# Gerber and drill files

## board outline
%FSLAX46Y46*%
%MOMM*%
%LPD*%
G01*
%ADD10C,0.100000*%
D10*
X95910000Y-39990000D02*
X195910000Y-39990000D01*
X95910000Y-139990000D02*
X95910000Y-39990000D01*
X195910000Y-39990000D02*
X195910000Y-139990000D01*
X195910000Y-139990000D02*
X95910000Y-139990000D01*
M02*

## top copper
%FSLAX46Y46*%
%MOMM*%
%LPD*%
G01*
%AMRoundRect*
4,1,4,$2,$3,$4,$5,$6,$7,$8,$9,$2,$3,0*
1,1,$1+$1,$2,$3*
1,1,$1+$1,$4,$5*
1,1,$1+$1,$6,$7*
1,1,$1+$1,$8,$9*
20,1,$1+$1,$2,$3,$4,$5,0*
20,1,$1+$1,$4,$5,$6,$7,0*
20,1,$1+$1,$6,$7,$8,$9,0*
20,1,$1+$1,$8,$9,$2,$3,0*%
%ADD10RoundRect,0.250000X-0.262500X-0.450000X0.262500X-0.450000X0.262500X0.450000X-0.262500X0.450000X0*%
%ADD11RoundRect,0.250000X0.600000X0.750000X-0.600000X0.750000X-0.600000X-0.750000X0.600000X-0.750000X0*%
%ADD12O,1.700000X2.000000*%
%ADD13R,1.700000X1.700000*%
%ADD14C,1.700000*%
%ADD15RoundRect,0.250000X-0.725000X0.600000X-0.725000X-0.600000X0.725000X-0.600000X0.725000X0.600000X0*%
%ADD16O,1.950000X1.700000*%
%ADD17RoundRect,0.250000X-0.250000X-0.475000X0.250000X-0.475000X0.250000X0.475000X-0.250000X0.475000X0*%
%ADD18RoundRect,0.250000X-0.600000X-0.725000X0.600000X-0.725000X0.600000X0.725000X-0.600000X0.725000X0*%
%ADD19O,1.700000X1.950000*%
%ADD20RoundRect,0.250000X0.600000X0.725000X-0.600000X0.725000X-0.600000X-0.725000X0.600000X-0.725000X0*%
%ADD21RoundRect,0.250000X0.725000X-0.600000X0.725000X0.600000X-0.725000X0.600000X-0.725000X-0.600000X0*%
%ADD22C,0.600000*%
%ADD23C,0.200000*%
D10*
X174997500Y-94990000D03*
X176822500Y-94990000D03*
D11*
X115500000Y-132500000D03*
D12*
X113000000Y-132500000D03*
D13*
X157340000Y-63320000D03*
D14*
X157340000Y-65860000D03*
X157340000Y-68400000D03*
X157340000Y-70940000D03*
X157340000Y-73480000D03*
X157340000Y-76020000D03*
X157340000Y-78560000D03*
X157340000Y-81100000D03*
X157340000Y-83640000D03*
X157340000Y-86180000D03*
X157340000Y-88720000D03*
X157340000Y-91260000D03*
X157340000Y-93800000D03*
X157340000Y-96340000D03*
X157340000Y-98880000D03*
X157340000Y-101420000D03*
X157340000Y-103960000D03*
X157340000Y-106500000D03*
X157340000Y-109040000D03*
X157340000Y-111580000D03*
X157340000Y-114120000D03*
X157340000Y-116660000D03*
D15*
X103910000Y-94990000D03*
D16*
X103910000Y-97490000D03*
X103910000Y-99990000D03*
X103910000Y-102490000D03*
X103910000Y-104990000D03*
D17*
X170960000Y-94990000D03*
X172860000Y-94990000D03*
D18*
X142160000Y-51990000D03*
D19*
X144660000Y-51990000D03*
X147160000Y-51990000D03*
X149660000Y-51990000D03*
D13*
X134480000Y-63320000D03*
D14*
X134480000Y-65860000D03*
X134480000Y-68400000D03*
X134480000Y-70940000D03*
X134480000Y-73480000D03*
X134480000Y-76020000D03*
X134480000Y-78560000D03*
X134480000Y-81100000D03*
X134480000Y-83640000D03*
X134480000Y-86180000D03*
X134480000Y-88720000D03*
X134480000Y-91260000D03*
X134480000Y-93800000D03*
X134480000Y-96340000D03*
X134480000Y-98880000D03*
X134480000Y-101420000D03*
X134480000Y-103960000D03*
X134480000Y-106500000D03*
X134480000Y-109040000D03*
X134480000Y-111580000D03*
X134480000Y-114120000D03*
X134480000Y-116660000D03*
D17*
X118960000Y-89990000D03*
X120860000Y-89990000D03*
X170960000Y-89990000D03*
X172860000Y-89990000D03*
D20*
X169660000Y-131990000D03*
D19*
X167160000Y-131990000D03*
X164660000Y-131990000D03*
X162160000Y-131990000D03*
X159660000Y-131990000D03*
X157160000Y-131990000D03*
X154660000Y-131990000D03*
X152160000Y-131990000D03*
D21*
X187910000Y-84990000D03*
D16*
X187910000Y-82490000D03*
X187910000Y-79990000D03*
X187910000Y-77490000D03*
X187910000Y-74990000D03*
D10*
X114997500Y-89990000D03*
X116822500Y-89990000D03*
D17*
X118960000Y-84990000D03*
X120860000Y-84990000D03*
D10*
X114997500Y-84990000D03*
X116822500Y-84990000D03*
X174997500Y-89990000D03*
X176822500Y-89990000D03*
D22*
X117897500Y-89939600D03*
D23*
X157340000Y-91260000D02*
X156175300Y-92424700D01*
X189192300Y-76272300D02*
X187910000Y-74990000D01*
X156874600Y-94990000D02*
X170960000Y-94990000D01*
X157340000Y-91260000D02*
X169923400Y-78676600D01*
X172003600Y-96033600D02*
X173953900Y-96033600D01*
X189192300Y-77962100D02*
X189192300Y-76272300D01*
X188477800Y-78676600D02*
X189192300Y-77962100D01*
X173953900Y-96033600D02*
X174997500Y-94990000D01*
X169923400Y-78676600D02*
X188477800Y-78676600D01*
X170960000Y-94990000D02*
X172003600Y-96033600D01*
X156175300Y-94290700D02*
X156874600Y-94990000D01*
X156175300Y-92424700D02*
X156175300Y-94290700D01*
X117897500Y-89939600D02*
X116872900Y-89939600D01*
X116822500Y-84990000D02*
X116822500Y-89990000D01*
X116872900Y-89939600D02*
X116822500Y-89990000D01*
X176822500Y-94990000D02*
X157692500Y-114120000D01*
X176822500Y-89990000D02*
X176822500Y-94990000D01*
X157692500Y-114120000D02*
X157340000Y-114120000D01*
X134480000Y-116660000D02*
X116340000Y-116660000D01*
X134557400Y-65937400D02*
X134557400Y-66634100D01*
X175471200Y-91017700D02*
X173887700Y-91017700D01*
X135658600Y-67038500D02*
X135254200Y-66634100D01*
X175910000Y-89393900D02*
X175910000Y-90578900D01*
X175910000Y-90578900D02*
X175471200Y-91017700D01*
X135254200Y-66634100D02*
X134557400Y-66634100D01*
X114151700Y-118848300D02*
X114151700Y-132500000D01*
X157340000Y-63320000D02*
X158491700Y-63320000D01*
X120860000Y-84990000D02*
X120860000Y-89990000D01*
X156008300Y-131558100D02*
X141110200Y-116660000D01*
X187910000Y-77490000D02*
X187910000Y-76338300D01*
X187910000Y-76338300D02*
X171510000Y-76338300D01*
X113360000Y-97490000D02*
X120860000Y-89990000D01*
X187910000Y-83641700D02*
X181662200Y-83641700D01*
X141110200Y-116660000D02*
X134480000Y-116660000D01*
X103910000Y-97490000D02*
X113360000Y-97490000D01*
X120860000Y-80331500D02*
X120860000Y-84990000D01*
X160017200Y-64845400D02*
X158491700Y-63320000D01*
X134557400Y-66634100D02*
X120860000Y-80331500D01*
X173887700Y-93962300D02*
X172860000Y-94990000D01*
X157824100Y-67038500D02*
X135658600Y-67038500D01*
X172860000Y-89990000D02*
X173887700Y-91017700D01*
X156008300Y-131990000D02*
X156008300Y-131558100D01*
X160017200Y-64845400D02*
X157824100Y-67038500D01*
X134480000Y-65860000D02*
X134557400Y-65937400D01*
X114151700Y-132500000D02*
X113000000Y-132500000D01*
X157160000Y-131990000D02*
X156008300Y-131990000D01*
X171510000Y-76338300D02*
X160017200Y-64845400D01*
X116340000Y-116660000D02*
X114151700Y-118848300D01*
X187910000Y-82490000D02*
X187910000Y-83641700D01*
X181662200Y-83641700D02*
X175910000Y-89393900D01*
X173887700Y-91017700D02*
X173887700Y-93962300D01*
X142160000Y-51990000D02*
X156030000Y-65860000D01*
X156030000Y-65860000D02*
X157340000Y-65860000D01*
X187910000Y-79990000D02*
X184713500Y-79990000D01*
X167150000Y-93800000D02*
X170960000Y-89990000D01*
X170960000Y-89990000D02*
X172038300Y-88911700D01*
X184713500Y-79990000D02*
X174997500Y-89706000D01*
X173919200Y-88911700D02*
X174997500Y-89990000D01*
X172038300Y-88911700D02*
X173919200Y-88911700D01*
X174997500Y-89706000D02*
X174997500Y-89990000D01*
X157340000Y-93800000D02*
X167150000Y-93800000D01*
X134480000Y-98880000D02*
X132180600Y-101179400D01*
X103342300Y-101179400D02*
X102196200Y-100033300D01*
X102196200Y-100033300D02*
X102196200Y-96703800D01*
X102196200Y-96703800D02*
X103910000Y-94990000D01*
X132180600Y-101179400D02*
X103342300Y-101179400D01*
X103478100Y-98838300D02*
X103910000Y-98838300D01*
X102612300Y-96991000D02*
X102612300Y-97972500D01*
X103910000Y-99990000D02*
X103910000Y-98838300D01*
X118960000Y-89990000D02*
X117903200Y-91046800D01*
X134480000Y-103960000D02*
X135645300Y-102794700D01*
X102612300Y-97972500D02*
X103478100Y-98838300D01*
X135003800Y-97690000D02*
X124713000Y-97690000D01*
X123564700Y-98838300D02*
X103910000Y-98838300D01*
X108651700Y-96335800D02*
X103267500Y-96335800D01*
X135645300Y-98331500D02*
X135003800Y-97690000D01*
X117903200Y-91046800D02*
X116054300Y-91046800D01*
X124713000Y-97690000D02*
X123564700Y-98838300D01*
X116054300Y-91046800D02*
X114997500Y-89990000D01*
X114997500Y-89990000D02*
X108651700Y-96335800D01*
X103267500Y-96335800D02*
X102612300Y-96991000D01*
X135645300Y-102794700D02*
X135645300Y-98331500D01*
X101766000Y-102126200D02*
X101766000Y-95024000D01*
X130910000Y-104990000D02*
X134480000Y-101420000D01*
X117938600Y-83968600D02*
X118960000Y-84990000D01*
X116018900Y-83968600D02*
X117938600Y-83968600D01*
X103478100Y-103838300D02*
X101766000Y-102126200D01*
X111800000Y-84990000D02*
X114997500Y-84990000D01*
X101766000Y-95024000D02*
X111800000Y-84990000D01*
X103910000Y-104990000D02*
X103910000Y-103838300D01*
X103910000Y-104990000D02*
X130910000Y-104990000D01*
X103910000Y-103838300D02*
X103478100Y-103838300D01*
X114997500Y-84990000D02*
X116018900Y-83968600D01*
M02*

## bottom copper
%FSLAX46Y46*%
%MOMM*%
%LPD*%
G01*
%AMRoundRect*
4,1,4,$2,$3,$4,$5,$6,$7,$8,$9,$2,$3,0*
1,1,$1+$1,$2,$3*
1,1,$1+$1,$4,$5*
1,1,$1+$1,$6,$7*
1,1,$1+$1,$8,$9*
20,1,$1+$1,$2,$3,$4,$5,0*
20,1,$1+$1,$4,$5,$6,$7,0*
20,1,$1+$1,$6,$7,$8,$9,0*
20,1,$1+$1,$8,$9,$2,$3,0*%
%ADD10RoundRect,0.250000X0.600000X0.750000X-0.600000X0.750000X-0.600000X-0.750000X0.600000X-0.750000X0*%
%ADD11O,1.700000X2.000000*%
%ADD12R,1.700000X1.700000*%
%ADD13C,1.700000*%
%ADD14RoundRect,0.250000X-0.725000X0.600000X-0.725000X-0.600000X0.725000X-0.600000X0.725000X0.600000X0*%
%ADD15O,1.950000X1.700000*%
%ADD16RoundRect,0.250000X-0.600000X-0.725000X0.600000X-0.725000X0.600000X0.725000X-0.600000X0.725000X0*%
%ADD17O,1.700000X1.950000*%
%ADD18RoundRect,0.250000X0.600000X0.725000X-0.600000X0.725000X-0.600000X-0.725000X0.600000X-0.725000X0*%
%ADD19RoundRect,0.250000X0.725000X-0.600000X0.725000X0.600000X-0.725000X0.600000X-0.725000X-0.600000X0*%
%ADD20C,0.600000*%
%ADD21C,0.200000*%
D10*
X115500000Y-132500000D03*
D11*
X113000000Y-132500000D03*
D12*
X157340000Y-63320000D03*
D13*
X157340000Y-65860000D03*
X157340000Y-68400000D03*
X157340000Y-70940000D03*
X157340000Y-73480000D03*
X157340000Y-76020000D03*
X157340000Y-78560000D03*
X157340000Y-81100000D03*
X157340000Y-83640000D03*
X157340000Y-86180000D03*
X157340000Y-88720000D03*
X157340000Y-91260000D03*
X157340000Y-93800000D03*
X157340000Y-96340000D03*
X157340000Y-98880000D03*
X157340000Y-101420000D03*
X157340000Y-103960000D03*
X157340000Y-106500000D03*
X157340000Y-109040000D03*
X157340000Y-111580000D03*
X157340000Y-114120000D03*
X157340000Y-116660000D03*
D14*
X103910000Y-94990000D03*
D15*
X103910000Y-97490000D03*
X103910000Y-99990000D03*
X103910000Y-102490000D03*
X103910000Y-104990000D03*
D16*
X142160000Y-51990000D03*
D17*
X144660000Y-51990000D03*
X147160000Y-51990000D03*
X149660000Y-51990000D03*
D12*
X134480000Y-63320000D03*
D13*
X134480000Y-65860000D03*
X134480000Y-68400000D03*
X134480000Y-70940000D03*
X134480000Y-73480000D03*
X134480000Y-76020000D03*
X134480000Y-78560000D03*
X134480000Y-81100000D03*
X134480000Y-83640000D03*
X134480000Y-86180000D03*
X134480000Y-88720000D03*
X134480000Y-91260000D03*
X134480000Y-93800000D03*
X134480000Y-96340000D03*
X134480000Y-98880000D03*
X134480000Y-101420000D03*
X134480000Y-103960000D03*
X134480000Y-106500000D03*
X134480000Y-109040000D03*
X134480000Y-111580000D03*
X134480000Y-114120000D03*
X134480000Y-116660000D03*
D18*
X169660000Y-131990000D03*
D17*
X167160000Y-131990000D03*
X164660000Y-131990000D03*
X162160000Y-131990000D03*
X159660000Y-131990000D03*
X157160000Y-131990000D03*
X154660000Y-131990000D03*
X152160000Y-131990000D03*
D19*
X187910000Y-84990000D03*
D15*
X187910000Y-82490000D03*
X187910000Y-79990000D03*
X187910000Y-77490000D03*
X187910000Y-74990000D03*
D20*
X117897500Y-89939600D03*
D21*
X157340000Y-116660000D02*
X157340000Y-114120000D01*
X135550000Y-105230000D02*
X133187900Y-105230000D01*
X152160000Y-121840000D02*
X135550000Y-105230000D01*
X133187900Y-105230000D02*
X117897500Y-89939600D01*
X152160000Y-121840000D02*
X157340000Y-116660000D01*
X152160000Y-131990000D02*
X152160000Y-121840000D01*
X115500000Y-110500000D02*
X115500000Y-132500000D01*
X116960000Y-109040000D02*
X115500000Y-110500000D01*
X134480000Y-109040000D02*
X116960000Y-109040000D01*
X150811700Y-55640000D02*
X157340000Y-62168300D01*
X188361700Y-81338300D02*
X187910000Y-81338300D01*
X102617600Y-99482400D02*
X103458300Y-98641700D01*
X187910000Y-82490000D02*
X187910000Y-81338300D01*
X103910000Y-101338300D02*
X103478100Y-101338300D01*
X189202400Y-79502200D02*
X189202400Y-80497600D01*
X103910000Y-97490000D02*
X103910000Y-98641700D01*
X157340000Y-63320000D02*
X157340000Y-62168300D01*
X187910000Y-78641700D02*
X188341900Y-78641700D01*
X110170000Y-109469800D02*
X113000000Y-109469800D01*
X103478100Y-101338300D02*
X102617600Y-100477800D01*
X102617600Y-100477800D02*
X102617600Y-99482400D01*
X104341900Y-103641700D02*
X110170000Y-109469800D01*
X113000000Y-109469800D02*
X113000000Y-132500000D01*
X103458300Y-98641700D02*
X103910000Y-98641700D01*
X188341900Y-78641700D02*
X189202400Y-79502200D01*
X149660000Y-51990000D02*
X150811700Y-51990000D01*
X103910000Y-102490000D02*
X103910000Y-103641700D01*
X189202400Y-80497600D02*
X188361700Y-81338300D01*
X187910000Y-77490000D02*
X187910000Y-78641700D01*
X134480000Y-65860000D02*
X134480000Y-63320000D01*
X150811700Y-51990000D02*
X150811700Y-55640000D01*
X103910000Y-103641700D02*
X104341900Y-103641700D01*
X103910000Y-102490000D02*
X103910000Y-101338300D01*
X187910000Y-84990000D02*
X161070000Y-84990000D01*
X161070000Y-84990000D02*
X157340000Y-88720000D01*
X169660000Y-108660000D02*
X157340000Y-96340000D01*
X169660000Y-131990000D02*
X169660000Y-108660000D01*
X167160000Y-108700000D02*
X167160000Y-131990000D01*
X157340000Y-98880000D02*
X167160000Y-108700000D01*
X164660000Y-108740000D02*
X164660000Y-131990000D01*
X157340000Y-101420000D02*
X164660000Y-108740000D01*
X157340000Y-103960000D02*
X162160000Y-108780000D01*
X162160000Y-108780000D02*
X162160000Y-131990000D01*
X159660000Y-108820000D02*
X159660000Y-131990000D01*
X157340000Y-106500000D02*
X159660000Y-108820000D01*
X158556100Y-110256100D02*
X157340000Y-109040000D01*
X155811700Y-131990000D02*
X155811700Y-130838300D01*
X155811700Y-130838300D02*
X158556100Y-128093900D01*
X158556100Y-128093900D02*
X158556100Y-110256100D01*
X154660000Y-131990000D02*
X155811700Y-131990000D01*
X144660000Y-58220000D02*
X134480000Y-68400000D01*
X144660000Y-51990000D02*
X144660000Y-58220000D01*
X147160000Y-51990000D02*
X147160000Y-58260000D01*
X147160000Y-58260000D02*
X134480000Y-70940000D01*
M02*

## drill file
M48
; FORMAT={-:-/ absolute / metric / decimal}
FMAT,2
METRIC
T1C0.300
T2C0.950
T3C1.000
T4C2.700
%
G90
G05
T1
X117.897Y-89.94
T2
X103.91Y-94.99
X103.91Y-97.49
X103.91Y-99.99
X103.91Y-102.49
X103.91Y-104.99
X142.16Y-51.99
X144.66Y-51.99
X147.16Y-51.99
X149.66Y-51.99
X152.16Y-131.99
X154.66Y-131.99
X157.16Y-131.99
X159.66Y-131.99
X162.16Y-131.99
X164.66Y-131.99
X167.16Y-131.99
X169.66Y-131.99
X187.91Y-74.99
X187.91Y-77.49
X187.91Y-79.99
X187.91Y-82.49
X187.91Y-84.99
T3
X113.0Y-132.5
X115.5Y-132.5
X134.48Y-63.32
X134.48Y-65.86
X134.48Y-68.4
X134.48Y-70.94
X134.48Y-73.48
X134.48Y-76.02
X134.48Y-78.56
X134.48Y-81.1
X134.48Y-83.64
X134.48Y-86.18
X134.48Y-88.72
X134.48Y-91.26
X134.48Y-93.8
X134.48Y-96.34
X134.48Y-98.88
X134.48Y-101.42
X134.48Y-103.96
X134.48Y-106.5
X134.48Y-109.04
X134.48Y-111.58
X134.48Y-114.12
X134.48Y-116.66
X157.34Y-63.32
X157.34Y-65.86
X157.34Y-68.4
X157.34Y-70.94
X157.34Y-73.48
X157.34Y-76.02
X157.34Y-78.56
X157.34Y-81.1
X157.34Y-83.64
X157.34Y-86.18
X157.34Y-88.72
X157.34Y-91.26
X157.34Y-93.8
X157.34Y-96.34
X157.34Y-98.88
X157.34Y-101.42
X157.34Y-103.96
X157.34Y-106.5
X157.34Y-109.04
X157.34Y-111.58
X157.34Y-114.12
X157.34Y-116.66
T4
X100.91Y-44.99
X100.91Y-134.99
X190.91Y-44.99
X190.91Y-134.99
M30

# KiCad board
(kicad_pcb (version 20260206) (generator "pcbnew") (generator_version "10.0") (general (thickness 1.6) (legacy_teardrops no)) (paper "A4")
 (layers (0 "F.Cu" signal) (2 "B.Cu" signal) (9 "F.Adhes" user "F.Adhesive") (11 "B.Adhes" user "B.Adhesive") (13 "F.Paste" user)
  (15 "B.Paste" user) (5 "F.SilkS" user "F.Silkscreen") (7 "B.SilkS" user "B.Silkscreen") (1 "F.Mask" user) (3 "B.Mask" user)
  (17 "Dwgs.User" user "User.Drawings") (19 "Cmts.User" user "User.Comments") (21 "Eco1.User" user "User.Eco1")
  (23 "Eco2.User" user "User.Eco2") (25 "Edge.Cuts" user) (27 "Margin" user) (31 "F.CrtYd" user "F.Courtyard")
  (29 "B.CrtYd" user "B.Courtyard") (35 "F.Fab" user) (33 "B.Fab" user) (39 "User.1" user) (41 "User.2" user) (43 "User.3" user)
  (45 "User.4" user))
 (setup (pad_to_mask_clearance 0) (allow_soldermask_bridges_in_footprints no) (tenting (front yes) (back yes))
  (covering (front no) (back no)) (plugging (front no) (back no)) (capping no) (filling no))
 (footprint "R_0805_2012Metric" (layer "F.Cu") (at 175.91 94.99)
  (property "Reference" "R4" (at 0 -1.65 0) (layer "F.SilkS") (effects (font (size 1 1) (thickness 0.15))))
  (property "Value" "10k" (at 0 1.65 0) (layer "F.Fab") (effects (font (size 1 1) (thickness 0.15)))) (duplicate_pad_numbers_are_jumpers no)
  (pad "1" smd roundrect (at -0.9125 0) (size 1.025 1.4) (layers "F.Cu" "F.Mask" "F.Paste") (roundrect_rratio 0.243902) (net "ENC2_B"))
  (pad "2" smd roundrect (at 0.9125 0) (size 1.025 1.4) (layers "F.Cu" "F.Mask" "F.Paste") (roundrect_rratio 0.243902) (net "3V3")))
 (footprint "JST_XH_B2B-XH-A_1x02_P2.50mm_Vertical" (layer "F.Cu") (at 115.5 132.5 180)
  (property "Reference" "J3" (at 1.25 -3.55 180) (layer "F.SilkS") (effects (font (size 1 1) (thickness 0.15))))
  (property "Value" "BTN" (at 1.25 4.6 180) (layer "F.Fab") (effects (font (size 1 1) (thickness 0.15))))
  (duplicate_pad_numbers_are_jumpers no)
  (pad "1" thru_hole roundrect (at 0 0 180) (size 1.7 2) (drill 1) (layers "*.Cu" "*.Mask") (remove_unused_layers no)
   (roundrect_rratio 0.147059) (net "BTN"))
  (pad "2" thru_hole oval (at 2.5 0 180) (size 1.7 2) (drill 1) (layers "*.Cu" "*.Mask") (remove_unused_layers no) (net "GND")))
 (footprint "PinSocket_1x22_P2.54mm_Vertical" (layer "F.Cu") (at 157.34 63.32)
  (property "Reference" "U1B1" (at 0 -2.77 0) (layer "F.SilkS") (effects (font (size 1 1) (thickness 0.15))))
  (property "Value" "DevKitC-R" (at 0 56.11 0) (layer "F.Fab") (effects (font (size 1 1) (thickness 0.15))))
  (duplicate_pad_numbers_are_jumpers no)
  (pad "1" thru_hole rect (at 0 0) (size 1.7 1.7) (drill 1) (layers "*.Cu" "*.Mask") (remove_unused_layers no) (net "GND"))
  (pad "2" thru_hole circle (at 0 2.54) (size 1.7 1.7) (drill 1) (layers "*.Cu" "*.Mask") (remove_unused_layers no) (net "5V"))
  (pad "3" thru_hole circle (at 0 5.08) (size 1.7 1.7) (drill 1) (layers "*.Cu" "*.Mask") (remove_unused_layers no))
  (pad "4" thru_hole circle (at 0 7.62) (size 1.7 1.7) (drill 1) (layers "*.Cu" "*.Mask") (remove_unused_layers no))
  (pad "5" thru_hole circle (at 0 10.16) (size 1.7 1.7) (drill 1) (layers "*.Cu" "*.Mask") (remove_unused_layers no))
  (pad "6" thru_hole circle (at 0 12.7) (size 1.7 1.7) (drill 1) (layers "*.Cu" "*.Mask") (remove_unused_layers no))
  (pad "7" thru_hole circle (at 0 15.24) (size 1.7 1.7) (drill 1) (layers "*.Cu" "*.Mask") (remove_unused_layers no))
  (pad "8" thru_hole circle (at 0 17.78) (size 1.7 1.7) (drill 1) (layers "*.Cu" "*.Mask") (remove_unused_layers no))
  (pad "9" thru_hole circle (at 0 20.32) (size 1.7 1.7) (drill 1) (layers "*.Cu" "*.Mask") (remove_unused_layers no))
  (pad "10" thru_hole circle (at 0 22.86) (size 1.7 1.7) (drill 1) (layers "*.Cu" "*.Mask") (remove_unused_layers no))
  (pad "11" thru_hole circle (at 0 25.4) (size 1.7 1.7) (drill 1) (layers "*.Cu" "*.Mask") (remove_unused_layers no) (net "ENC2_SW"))
  (pad "12" thru_hole circle (at 0 27.94) (size 1.7 1.7) (drill 1) (layers "*.Cu" "*.Mask") (remove_unused_layers no) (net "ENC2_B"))
  (pad "13" thru_hole circle (at 0 30.48) (size 1.7 1.7) (drill 1) (layers "*.Cu" "*.Mask") (remove_unused_layers no) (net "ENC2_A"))
  (pad "14" thru_hole circle (at 0 33.02) (size 1.7 1.7) (drill 1) (layers "*.Cu" "*.Mask") (remove_unused_layers no) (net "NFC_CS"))
  (pad "15" thru_hole circle (at 0 35.56) (size 1.7 1.7) (drill 1) (layers "*.Cu" "*.Mask") (remove_unused_layers no) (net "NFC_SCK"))
  (pad "16" thru_hole circle (at 0 38.1) (size 1.7 1.7) (drill 1) (layers "*.Cu" "*.Mask") (remove_unused_layers no) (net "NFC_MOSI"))
  (pad "17" thru_hole circle (at 0 40.64) (size 1.7 1.7) (drill 1) (layers "*.Cu" "*.Mask") (remove_unused_layers no) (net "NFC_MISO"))
  (pad "18" thru_hole circle (at 0 43.18) (size 1.7 1.7) (drill 1) (layers "*.Cu" "*.Mask") (remove_unused_layers no) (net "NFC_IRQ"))
  (pad "19" thru_hole circle (at 0 45.72) (size 1.7 1.7) (drill 1) (layers "*.Cu" "*.Mask") (remove_unused_layers no) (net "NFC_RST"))
  (pad "20" thru_hole circle (at 0 48.26) (size 1.7 1.7) (drill 1) (layers "*.Cu" "*.Mask") (remove_unused_layers no))
  (pad "21" thru_hole circle (at 0 50.8) (size 1.7 1.7) (drill 1) (layers "*.Cu" "*.Mask") (remove_unused_layers no) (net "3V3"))
  (pad "22" thru_hole circle (at 0 53.34) (size 1.7 1.7) (drill 1) (layers "*.Cu" "*.Mask") (remove_unused_layers no) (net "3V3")))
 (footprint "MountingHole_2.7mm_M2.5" (layer "F.Cu") (at 190.91 44.99)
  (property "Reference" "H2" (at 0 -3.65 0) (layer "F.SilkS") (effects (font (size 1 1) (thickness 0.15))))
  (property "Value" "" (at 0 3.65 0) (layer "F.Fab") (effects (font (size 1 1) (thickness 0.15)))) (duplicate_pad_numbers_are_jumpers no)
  (pad "" np_thru_hole circle (at 0 0) (size 2.7 2.7) (drill 2.7) (layers "*.Cu" "*.Mask")))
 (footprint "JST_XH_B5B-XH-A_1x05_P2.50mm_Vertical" (layer "F.Cu") (at 103.91 94.99 -90)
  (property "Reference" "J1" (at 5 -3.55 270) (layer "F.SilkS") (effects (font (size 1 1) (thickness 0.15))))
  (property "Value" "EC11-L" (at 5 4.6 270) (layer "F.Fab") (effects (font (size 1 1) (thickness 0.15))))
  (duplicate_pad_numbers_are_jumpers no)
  (pad "1" thru_hole roundrect (at 0 0 270) (size 1.7 1.95) (drill 0.95) (layers "*.Cu" "*.Mask") (remove_unused_layers no)
   (roundrect_rratio 0.147059) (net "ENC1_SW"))
  (pad "2" thru_hole oval (at 2.5 0 270) (size 1.7 1.95) (drill 0.95) (layers "*.Cu" "*.Mask") (remove_unused_layers no) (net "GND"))
  (pad "3" thru_hole oval (at 5 0 270) (size 1.7 1.95) (drill 0.95) (layers "*.Cu" "*.Mask") (remove_unused_layers no) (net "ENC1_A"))
  (pad "4" thru_hole oval (at 7.5 0 270) (size 1.7 1.95) (drill 0.95) (layers "*.Cu" "*.Mask") (remove_unused_layers no) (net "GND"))
  (pad "5" thru_hole oval (at 10 0 270) (size 1.7 1.95) (drill 0.95) (layers "*.Cu" "*.Mask") (remove_unused_layers no) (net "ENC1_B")))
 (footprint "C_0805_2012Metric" (layer "F.Cu") (at 171.91 94.99)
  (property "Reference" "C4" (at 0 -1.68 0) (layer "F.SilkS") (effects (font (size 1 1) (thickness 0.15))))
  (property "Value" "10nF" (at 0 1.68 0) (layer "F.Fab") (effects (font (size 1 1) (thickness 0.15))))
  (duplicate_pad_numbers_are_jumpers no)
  (pad "1" smd roundrect (at -0.95 0) (size 1 1.45) (layers "F.Cu" "F.Mask" "F.Paste") (roundrect_rratio 0.25) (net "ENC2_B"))
  (pad "2" smd roundrect (at 0.95 0) (size 1 1.45) (layers "F.Cu" "F.Mask" "F.Paste") (roundrect_rratio 0.25) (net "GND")))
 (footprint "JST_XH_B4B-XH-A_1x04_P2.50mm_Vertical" (layer "F.Cu") (at 142.16 51.99)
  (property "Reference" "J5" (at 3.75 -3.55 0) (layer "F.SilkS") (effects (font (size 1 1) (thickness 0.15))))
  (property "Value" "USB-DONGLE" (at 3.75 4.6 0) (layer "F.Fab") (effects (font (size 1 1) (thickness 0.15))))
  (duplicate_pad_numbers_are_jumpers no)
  (pad "1" thru_hole roundrect (at 0 0) (size 1.7 1.95) (drill 0.95) (layers "*.Cu" "*.Mask") (remove_unused_layers no)
   (roundrect_rratio 0.147059) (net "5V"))
  (pad "2" thru_hole oval (at 2.5 0) (size 1.7 1.95) (drill 0.95) (layers "*.Cu" "*.Mask") (remove_unused_layers no) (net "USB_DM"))
  (pad "3" thru_hole oval (at 5 0) (size 1.7 1.95) (drill 0.95) (layers "*.Cu" "*.Mask") (remove_unused_layers no) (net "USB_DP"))
  (pad "4" thru_hole oval (at 7.5 0) (size 1.7 1.95) (drill 0.95) (layers "*.Cu" "*.Mask") (remove_unused_layers no) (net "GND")))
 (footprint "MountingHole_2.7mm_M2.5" (layer "F.Cu") (at 100.91 134.99)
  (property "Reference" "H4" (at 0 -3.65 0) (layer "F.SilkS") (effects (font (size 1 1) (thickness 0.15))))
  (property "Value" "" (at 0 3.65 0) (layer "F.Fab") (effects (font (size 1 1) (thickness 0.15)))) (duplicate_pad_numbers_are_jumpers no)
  (pad "" np_thru_hole circle (at 0 0) (size 2.7 2.7) (drill 2.7) (layers "*.Cu" "*.Mask")))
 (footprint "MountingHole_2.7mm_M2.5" (layer "F.Cu") (at 100.91 44.99)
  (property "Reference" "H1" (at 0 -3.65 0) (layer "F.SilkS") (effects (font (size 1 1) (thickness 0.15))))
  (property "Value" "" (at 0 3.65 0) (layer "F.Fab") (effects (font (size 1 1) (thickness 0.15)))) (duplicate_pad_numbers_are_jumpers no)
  (pad "" np_thru_hole circle (at 0 0) (size 2.7 2.7) (drill 2.7) (layers "*.Cu" "*.Mask")))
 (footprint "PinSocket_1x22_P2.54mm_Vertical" (layer "F.Cu") (at 134.48 63.32)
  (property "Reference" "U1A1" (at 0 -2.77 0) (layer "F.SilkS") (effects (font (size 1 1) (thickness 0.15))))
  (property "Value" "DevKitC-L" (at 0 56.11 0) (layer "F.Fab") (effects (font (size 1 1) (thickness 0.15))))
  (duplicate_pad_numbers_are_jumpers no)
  (pad "1" thru_hole rect (at 0 0) (size 1.7 1.7) (drill 1) (layers "*.Cu" "*.Mask") (remove_unused_layers no) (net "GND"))
  (pad "2" thru_hole circle (at 0 2.54) (size 1.7 1.7) (drill 1) (layers "*.Cu" "*.Mask") (remove_unused_layers no) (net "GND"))
  (pad "3" thru_hole circle (at 0 5.08) (size 1.7 1.7) (drill 1) (layers "*.Cu" "*.Mask") (remove_unused_layers no) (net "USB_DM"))
  (pad "4" thru_hole circle (at 0 7.62) (size 1.7 1.7) (drill 1) (layers "*.Cu" "*.Mask") (remove_unused_layers no) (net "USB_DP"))
  (pad "5" thru_hole circle (at 0 10.16) (size 1.7 1.7) (drill 1) (layers "*.Cu" "*.Mask") (remove_unused_layers no))
  (pad "6" thru_hole circle (at 0 12.7) (size 1.7 1.7) (drill 1) (layers "*.Cu" "*.Mask") (remove_unused_layers no))
  (pad "7" thru_hole circle (at 0 15.24) (size 1.7 1.7) (drill 1) (layers "*.Cu" "*.Mask") (remove_unused_layers no))
  (pad "8" thru_hole circle (at 0 17.78) (size 1.7 1.7) (drill 1) (layers "*.Cu" "*.Mask") (remove_unused_layers no))
  (pad "9" thru_hole circle (at 0 20.32) (size 1.7 1.7) (drill 1) (layers "*.Cu" "*.Mask") (remove_unused_layers no))
  (pad "10" thru_hole circle (at 0 22.86) (size 1.7 1.7) (drill 1) (layers "*.Cu" "*.Mask") (remove_unused_layers no))
  (pad "11" thru_hole circle (at 0 25.4) (size 1.7 1.7) (drill 1) (layers "*.Cu" "*.Mask") (remove_unused_layers no))
  (pad "12" thru_hole circle (at 0 27.94) (size 1.7 1.7) (drill 1) (layers "*.Cu" "*.Mask") (remove_unused_layers no))
  (pad "13" thru_hole circle (at 0 30.48) (size 1.7 1.7) (drill 1) (layers "*.Cu" "*.Mask") (remove_unused_layers no))
  (pad "14" thru_hole circle (at 0 33.02) (size 1.7 1.7) (drill 1) (layers "*.Cu" "*.Mask") (remove_unused_layers no))
  (pad "15" thru_hole circle (at 0 35.56) (size 1.7 1.7) (drill 1) (layers "*.Cu" "*.Mask") (remove_unused_layers no) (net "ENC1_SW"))
  (pad "16" thru_hole circle (at 0 38.1) (size 1.7 1.7) (drill 1) (layers "*.Cu" "*.Mask") (remove_unused_layers no) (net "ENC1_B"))
  (pad "17" thru_hole circle (at 0 40.64) (size 1.7 1.7) (drill 1) (layers "*.Cu" "*.Mask") (remove_unused_layers no) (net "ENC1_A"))
  (pad "18" thru_hole circle (at 0 43.18) (size 1.7 1.7) (drill 1) (layers "*.Cu" "*.Mask") (remove_unused_layers no))
  (pad "19" thru_hole circle (at 0 45.72) (size 1.7 1.7) (drill 1) (layers "*.Cu" "*.Mask") (remove_unused_layers no) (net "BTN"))
  (pad "20" thru_hole circle (at 0 48.26) (size 1.7 1.7) (drill 1) (layers "*.Cu" "*.Mask") (remove_unused_layers no))
  (pad "21" thru_hole circle (at 0 50.8) (size 1.7 1.7) (drill 1) (layers "*.Cu" "*.Mask") (remove_unused_layers no))
  (pad "22" thru_hole circle (at 0 53.34) (size 1.7 1.7) (drill 1) (layers "*.Cu" "*.Mask") (remove_unused_layers no) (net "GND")))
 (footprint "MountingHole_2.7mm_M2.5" (layer "F.Cu") (at 190.91 134.99)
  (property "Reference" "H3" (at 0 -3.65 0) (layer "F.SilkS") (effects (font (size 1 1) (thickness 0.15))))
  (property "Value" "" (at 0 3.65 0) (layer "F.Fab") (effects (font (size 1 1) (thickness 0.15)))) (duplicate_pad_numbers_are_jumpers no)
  (pad "" np_thru_hole circle (at 0 0) (size 2.7 2.7) (drill 2.7) (layers "*.Cu" "*.Mask")))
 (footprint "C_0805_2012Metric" (layer "F.Cu") (at 119.91 89.99)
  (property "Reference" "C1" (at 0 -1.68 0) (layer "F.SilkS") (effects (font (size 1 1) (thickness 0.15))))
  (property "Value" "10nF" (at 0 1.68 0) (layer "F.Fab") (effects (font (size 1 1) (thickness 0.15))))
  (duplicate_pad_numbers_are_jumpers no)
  (pad "1" smd roundrect (at -0.95 0) (size 1 1.45) (layers "F.Cu" "F.Mask" "F.Paste") (roundrect_rratio 0.25) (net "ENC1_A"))
  (pad "2" smd roundrect (at 0.95 0) (size 1 1.45) (layers "F.Cu" "F.Mask" "F.Paste") (roundrect_rratio 0.25) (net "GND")))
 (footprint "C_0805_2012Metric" (layer "F.Cu") (at 171.91 89.99)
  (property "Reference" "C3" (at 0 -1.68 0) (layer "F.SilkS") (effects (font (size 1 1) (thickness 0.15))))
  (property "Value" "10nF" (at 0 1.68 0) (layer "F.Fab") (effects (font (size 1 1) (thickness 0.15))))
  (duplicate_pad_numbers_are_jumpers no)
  (pad "1" smd roundrect (at -0.95 0) (size 1 1.45) (layers "F.Cu" "F.Mask" "F.Paste") (roundrect_rratio 0.25) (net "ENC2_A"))
  (pad "2" smd roundrect (at 0.95 0) (size 1 1.45) (layers "F.Cu" "F.Mask" "F.Paste") (roundrect_rratio 0.25) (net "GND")))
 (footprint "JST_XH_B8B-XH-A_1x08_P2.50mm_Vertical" (layer "F.Cu") (at 169.66 131.99 180)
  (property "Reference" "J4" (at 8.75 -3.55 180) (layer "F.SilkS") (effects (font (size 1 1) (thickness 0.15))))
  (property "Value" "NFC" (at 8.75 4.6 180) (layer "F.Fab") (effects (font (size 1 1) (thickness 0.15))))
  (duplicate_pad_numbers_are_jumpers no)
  (pad "1" thru_hole roundrect (at 0 0 180) (size 1.7 1.95) (drill 0.95) (layers "*.Cu" "*.Mask") (remove_unused_layers no)
   (roundrect_rratio 0.147059) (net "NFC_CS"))
  (pad "2" thru_hole oval (at 2.5 0 180) (size 1.7 1.95) (drill 0.95) (layers "*.Cu" "*.Mask") (remove_unused_layers no) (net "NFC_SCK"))
  (pad "3" thru_hole oval (at 5 0 180) (size 1.7 1.95) (drill 0.95) (layers "*.Cu" "*.Mask") (remove_unused_layers no) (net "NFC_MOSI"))
  (pad "4" thru_hole oval (at 7.5 0 180) (size 1.7 1.95) (drill 0.95) (layers "*.Cu" "*.Mask") (remove_unused_layers no) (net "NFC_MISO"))
  (pad "5" thru_hole oval (at 10 0 180) (size 1.7 1.95) (drill 0.95) (layers "*.Cu" "*.Mask") (remove_unused_layers no) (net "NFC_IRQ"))
  (pad "6" thru_hole oval (at 12.5 0 180) (size 1.7 1.95) (drill 0.95) (layers "*.Cu" "*.Mask") (remove_unused_layers no) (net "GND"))
  (pad "7" thru_hole oval (at 15 0 180) (size 1.7 1.95) (drill 0.95) (layers "*.Cu" "*.Mask") (remove_unused_layers no) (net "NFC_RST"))
  (pad "8" thru_hole oval (at 17.5 0 180) (size 1.7 1.95) (drill 0.95) (layers "*.Cu" "*.Mask") (remove_unused_layers no) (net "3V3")))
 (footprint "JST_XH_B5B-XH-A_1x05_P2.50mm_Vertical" (layer "F.Cu") (at 187.91 84.99 90)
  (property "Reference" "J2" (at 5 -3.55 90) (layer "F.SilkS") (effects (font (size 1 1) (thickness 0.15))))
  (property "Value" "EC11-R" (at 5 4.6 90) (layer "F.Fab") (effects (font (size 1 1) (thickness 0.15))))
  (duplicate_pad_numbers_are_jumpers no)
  (pad "1" thru_hole roundrect (at 0 0 90) (size 1.7 1.95) (drill 0.95) (layers "*.Cu" "*.Mask") (remove_unused_layers no)
   (roundrect_rratio 0.147059) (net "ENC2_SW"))
  (pad "2" thru_hole oval (at 2.5 0 90) (size 1.7 1.95) (drill 0.95) (layers "*.Cu" "*.Mask") (remove_unused_layers no) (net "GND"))
  (pad "3" thru_hole oval (at 5 0 90) (size 1.7 1.95) (drill 0.95) (layers "*.Cu" "*.Mask") (remove_unused_layers no) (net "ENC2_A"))
  (pad "4" thru_hole oval (at 7.5 0 90) (size 1.7 1.95) (drill 0.95) (layers "*.Cu" "*.Mask") (remove_unused_layers no) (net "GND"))
  (pad "5" thru_hole oval (at 10 0 90) (size 1.7 1.95) (drill 0.95) (layers "*.Cu" "*.Mask") (remove_unused_layers no) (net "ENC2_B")))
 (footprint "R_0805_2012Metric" (layer "F.Cu") (at 115.91 89.99)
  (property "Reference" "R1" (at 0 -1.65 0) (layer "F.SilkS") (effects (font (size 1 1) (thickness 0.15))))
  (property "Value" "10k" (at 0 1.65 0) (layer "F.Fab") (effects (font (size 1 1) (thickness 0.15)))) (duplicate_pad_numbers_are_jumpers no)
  (pad "1" smd roundrect (at -0.9125 0) (size 1.025 1.4) (layers "F.Cu" "F.Mask" "F.Paste") (roundrect_rratio 0.243902) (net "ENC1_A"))
  (pad "2" smd roundrect (at 0.9125 0) (size 1.025 1.4) (layers "F.Cu" "F.Mask" "F.Paste") (roundrect_rratio 0.243902) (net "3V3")))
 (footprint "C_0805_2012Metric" (layer "F.Cu") (at 119.91 84.99)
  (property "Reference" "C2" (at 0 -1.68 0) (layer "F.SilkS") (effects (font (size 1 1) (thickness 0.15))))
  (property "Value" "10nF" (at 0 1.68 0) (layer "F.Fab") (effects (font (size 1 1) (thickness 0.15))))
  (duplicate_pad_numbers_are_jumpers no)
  (pad "1" smd roundrect (at -0.95 0) (size 1 1.45) (layers "F.Cu" "F.Mask" "F.Paste") (roundrect_rratio 0.25) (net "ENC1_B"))
  (pad "2" smd roundrect (at 0.95 0) (size 1 1.45) (layers "F.Cu" "F.Mask" "F.Paste") (roundrect_rratio 0.25) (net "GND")))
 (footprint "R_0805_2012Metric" (layer "F.Cu") (at 115.91 84.99)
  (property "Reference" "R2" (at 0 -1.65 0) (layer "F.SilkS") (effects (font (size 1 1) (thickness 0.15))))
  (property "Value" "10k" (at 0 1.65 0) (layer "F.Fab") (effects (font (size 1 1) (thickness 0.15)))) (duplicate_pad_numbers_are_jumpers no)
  (pad "1" smd roundrect (at -0.9125 0) (size 1.025 1.4) (layers "F.Cu" "F.Mask" "F.Paste") (roundrect_rratio 0.243902) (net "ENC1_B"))
  (pad "2" smd roundrect (at 0.9125 0) (size 1.025 1.4) (layers "F.Cu" "F.Mask" "F.Paste") (roundrect_rratio 0.243902) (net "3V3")))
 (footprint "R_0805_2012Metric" (layer "F.Cu") (at 175.91 89.99)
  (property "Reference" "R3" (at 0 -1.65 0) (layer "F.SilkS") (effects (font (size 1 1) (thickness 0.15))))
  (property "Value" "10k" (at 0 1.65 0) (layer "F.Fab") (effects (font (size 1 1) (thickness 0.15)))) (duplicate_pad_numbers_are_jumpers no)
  (pad "1" smd roundrect (at -0.9125 0) (size 1.025 1.4) (layers "F.Cu" "F.Mask" "F.Paste") (roundrect_rratio 0.243902) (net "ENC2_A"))
  (pad "2" smd roundrect (at 0.9125 0) (size 1.025 1.4) (layers "F.Cu" "F.Mask" "F.Paste") (roundrect_rratio 0.243902) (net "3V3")))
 (gr_line (start 95.91 39.99) (end 195.91 39.99) (stroke (width 0.1) (type default)) (layer "Edge.Cuts"))
 (gr_line (start 95.91 139.99) (end 95.91 39.99) (stroke (width 0.1) (type default)) (layer "Edge.Cuts"))
 (gr_line (start 195.91 39.99) (end 195.91 139.99) (stroke (width 0.1) (type default)) (layer "Edge.Cuts"))
 (gr_line (start 195.91 139.99) (end 95.91 139.99) (stroke (width 0.1) (type default)) (layer "Edge.Cuts"))
 (segment (start 157.34 91.26) (end 156.1753 92.4247) (width 0.2) (layer "F.Cu") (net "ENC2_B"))
 (segment (start 189.1923 76.2723) (end 187.91 74.99) (width 0.2) (layer "F.Cu") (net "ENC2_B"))
 (segment (start 156.8746 94.99) (end 170.96 94.99) (width 0.2) (layer "F.Cu") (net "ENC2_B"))
 (segment (start 157.34 91.26) (end 169.9234 78.6766) (width 0.2) (layer "F.Cu") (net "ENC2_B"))
 (segment (start 172.0036 96.0336) (end 173.9539 96.0336) (width 0.2) (layer "F.Cu") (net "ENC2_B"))
 (segment (start 189.1923 77.9621) (end 189.1923 76.2723) (width 0.2) (layer "F.Cu") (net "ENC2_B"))
 (segment (start 188.4778 78.6766) (end 189.1923 77.9621) (width 0.2) (layer "F.Cu") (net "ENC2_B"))
 (segment (start 173.9539 96.0336) (end 174.9975 94.99) (width 0.2) (layer "F.Cu") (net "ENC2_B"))
 (segment (start 169.9234 78.6766) (end 188.4778 78.6766) (width 0.2) (layer "F.Cu") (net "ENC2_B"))
 (segment (start 170.96 94.99) (end 172.0036 96.0336) (width 0.2) (layer "F.Cu") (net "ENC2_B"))
 (segment (start 156.1753 94.2907) (end 156.8746 94.99) (width 0.2) (layer "F.Cu") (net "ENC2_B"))
 (segment (start 156.1753 92.4247) (end 156.1753 94.2907) (width 0.2) (layer "F.Cu") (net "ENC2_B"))
 (segment (start 117.8975 89.9396) (end 116.8729 89.9396) (width 0.2) (layer "F.Cu") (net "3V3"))
 (segment (start 116.8225 84.99) (end 116.8225 89.99) (width 0.2) (layer "F.Cu") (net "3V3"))
 (segment (start 116.8729 89.9396) (end 116.8225 89.99) (width 0.2) (layer "F.Cu") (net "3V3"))
 (segment (start 176.8225 94.99) (end 157.6925 114.12) (width 0.2) (layer "F.Cu") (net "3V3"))
 (segment (start 176.8225 89.99) (end 176.8225 94.99) (width 0.2) (layer "F.Cu") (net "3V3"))
 (segment (start 157.6925 114.12) (end 157.34 114.12) (width 0.2) (layer "F.Cu") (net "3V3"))
 (via (at 117.8975 89.9396) (size 0.6) (drill 0.3) (layers "F.Cu" "B.Cu") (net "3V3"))
 (segment (start 157.34 116.66) (end 157.34 114.12) (width 0.2) (layer "B.Cu") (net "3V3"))
 (segment (start 135.55 105.23) (end 133.1879 105.23) (width 0.2) (layer "B.Cu") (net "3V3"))
 (segment (start 152.16 121.84) (end 135.55 105.23) (width 0.2) (layer "B.Cu") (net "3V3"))
 (segment (start 133.1879 105.23) (end 117.8975 89.9396) (width 0.2) (layer "B.Cu") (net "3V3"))
 (segment (start 152.16 121.84) (end 157.34 116.66) (width 0.2) (layer "B.Cu") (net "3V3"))
 (segment (start 152.16 131.99) (end 152.16 121.84) (width 0.2) (layer "B.Cu") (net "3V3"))
 (segment (start 115.5 110.5) (end 115.5 132.5) (width 0.2) (layer "B.Cu") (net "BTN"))
 (segment (start 116.96 109.04) (end 115.5 110.5) (width 0.2) (layer "B.Cu") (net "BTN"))
 (segment (start 134.48 109.04) (end 116.96 109.04) (width 0.2) (layer "B.Cu") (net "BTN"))
 (segment (start 134.48 116.66) (end 116.34 116.66) (width 0.2) (layer "F.Cu") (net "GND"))
 (segment (start 134.5574 65.9374) (end 134.5574 66.6341) (width 0.2) (layer "F.Cu") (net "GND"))
 (segment (start 175.4712 91.0177) (end 173.8877 91.0177) (width 0.2) (layer "F.Cu") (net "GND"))
 (segment (start 135.6586 67.0385) (end 135.2542 66.6341) (width 0.2) (layer "F.Cu") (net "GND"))
 (segment (start 175.91 89.3939) (end 175.91 90.5789) (width 0.2) (layer "F.Cu") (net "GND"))
 (segment (start 175.91 90.5789) (end 175.4712 91.0177) (width 0.2) (layer "F.Cu") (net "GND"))
 (segment (start 135.2542 66.6341) (end 134.5574 66.6341) (width 0.2) (layer "F.Cu") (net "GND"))
 (segment (start 114.1517 118.8483) (end 114.1517 132.5) (width 0.2) (layer "F.Cu") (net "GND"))
 (segment (start 157.34 63.32) (end 158.4917 63.32) (width 0.2) (layer "F.Cu") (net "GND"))
 (segment (start 120.86 84.99) (end 120.86 89.99) (width 0.2) (layer "F.Cu") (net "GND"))
 (segment (start 156.0083 131.5581) (end 141.1102 116.66) (width 0.2) (layer "F.Cu") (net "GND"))
 (segment (start 187.91 77.49) (end 187.91 76.3383) (width 0.2) (layer "F.Cu") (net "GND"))
 (segment (start 187.91 76.3383) (end 171.51 76.3383) (width 0.2) (layer "F.Cu") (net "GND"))
 (segment (start 113.36 97.49) (end 120.86 89.99) (width 0.2) (layer "F.Cu") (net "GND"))
 (segment (start 187.91 83.6417) (end 181.6622 83.6417) (width 0.2) (layer "F.Cu") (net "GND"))
 (segment (start 141.1102 116.66) (end 134.48 116.66) (width 0.2) (layer "F.Cu") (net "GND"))
 (segment (start 103.91 97.49) (end 113.36 97.49) (width 0.2) (layer "F.Cu") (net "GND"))
 (segment (start 120.86 80.3315) (end 120.86 84.99) (width 0.2) (layer "F.Cu") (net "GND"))
 (segment (start 160.0172 64.8454) (end 158.4917 63.32) (width 0.2) (layer "F.Cu") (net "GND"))
 (segment (start 134.5574 66.6341) (end 120.86 80.3315) (width 0.2) (layer "F.Cu") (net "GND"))
 (segment (start 173.8877 93.9623) (end 172.86 94.99) (width 0.2) (layer "F.Cu") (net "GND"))
 (segment (start 157.8241 67.0385) (end 135.6586 67.0385) (width 0.2) (layer "F.Cu") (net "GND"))
 (segment (start 172.86 89.99) (end 173.8877 91.0177) (width 0.2) (layer "F.Cu") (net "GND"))
 (segment (start 156.0083 131.99) (end 156.0083 131.5581) (width 0.2) (layer "F.Cu") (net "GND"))
 (segment (start 160.0172 64.8454) (end 157.8241 67.0385) (width 0.2) (layer "F.Cu") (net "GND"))
 (segment (start 134.48 65.86) (end 134.5574 65.9374) (width 0.2) (layer "F.Cu") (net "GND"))
 (segment (start 114.1517 132.5) (end 113 132.5) (width 0.2) (layer "F.Cu") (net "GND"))
 (segment (start 157.16 131.99) (end 156.0083 131.99) (width 0.2) (layer "F.Cu") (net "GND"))
 (segment (start 171.51 76.3383) (end 160.0172 64.8454) (width 0.2) (layer "F.Cu") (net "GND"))
 (segment (start 116.34 116.66) (end 114.1517 118.8483) (width 0.2) (layer "F.Cu") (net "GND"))
 (segment (start 187.91 82.49) (end 187.91 83.6417) (width 0.2) (layer "F.Cu") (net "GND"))
 (segment (start 181.6622 83.6417) (end 175.91 89.3939) (width 0.2) (layer "F.Cu") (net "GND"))
 (segment (start 173.8877 91.0177) (end 173.8877 93.9623) (width 0.2) (layer "F.Cu") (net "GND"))
 (segment (start 150.8117 55.64) (end 157.34 62.1683) (width 0.2) (layer "B.Cu") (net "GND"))
 (segment (start 188.3617 81.3383) (end 187.91 81.3383) (width 0.2) (layer "B.Cu") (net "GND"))
 (segment (start 102.6176 99.4824) (end 103.4583 98.6417) (width 0.2) (layer "B.Cu") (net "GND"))
 (segment (start 187.91 82.49) (end 187.91 81.3383) (width 0.2) (layer "B.Cu") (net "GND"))
 (segment (start 103.91 101.3383) (end 103.4781 101.3383) (width 0.2) (layer "B.Cu") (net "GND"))
 (segment (start 189.2024 79.5022) (end 189.2024 80.4976) (width 0.2) (layer "B.Cu") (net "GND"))
 (segment (start 103.91 97.49) (end 103.91 98.6417) (width 0.2) (layer "B.Cu") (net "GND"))
 (segment (start 157.34 63.32) (end 157.34 62.1683) (width 0.2) (layer "B.Cu") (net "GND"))
 (segment (start 187.91 78.6417) (end 188.3419 78.6417) (width 0.2) (layer "B.Cu") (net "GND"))
 (segment (start 110.17 109.4698) (end 113 109.4698) (width 0.2) (layer "B.Cu") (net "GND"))
 (segment (start 103.4781 101.3383) (end 102.6176 100.4778) (width 0.2) (layer "B.Cu") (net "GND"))
 (segment (start 102.6176 100.4778) (end 102.6176 99.4824) (width 0.2) (layer "B.Cu") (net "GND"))
 (segment (start 104.3419 103.6417) (end 110.17 109.4698) (width 0.2) (layer "B.Cu") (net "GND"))
 (segment (start 113 109.4698) (end 113 132.5) (width 0.2) (layer "B.Cu") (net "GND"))
 (segment (start 103.4583 98.6417) (end 103.91 98.6417) (width 0.2) (layer "B.Cu") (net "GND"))
 (segment (start 188.3419 78.6417) (end 189.2024 79.5022) (width 0.2) (layer "B.Cu") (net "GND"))
 (segment (start 149.66 51.99) (end 150.8117 51.99) (width 0.2) (layer "B.Cu") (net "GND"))
 (segment (start 103.91 102.49) (end 103.91 103.6417) (width 0.2) (layer "B.Cu") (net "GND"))
 (segment (start 189.2024 80.4976) (end 188.3617 81.3383) (width 0.2) (layer "B.Cu") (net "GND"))
 (segment (start 187.91 77.49) (end 187.91 78.6417) (width 0.2) (layer "B.Cu") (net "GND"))
 (segment (start 134.48 65.86) (end 134.48 63.32) (width 0.2) (layer "B.Cu") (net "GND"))
 (segment (start 150.8117 51.99) (end 150.8117 55.64) (width 0.2) (layer "B.Cu") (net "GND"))
 (segment (start 103.91 103.6417) (end 104.3419 103.6417) (width 0.2) (layer "B.Cu") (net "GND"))
 (segment (start 103.91 102.49) (end 103.91 101.3383) (width 0.2) (layer "B.Cu") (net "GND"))
 (segment (start 142.16 51.99) (end 156.03 65.86) (width 0.2) (layer "F.Cu") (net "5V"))
 (segment (start 156.03 65.86) (end 157.34 65.86) (width 0.2) (layer "F.Cu") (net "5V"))
 (segment (start 187.91 84.99) (end 161.07 84.99) (width 0.2) (layer "B.Cu") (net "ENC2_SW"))
 (segment (start 161.07 84.99) (end 157.34 88.72) (width 0.2) (layer "B.Cu") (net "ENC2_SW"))
 (segment (start 187.91 79.99) (end 184.7135 79.99) (width 0.2) (layer "F.Cu") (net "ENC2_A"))
 (segment (start 167.15 93.8) (end 170.96 89.99) (width 0.2) (layer "F.Cu") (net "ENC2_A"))
 (segment (start 170.96 89.99) (end 172.0383 88.9117) (width 0.2) (layer "F.Cu") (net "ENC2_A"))
 (segment (start 184.7135 79.99) (end 174.9975 89.706) (width 0.2) (layer "F.Cu") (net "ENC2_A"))
 (segment (start 173.9192 88.9117) (end 174.9975 89.99) (width 0.2) (layer "F.Cu") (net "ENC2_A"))
 (segment (start 172.0383 88.9117) (end 173.9192 88.9117) (width 0.2) (layer "F.Cu") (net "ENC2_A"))
 (segment (start 174.9975 89.706) (end 174.9975 89.99) (width 0.2) (layer "F.Cu") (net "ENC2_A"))
 (segment (start 157.34 93.8) (end 167.15 93.8) (width 0.2) (layer "F.Cu") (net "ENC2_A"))
 (segment (start 169.66 108.66) (end 157.34 96.34) (width 0.2) (layer "B.Cu") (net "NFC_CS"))
 (segment (start 169.66 131.99) (end 169.66 108.66) (width 0.2) (layer "B.Cu") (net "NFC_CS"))
 (segment (start 167.16 108.7) (end 167.16 131.99) (width 0.2) (layer "B.Cu") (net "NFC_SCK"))
 (segment (start 157.34 98.88) (end 167.16 108.7) (width 0.2) (layer "B.Cu") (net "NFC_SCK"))
 (segment (start 164.66 108.74) (end 164.66 131.99) (width 0.2) (layer "B.Cu") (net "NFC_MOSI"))
 (segment (start 157.34 101.42) (end 164.66 108.74) (width 0.2) (layer "B.Cu") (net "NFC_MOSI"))
 (segment (start 157.34 103.96) (end 162.16 108.78) (width 0.2) (layer "B.Cu") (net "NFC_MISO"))
 (segment (start 162.16 108.78) (end 162.16 131.99) (width 0.2) (layer "B.Cu") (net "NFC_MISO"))
 (segment (start 159.66 108.82) (end 159.66 131.99) (width 0.2) (layer "B.Cu") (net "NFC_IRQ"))
 (segment (start 157.34 106.5) (end 159.66 108.82) (width 0.2) (layer "B.Cu") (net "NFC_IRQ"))
 (segment (start 158.5561 110.2561) (end 157.34 109.04) (width 0.2) (layer "B.Cu") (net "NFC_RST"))
 (segment (start 155.8117 131.99) (end 155.8117 130.8383) (width 0.2) (layer "B.Cu") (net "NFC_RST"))
 (segment (start 155.8117 130.8383) (end 158.5561 128.0939) (width 0.2) (layer "B.Cu") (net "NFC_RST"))
 (segment (start 158.5561 128.0939) (end 158.5561 110.2561) (width 0.2) (layer "B.Cu") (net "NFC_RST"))
 (segment (start 154.66 131.99) (end 155.8117 131.99) (width 0.2) (layer "B.Cu") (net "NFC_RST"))
 (segment (start 134.48 98.88) (end 132.1806 101.1794) (width 0.2) (layer "F.Cu") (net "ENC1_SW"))
 (segment (start 103.3423 101.1794) (end 102.1962 100.0333) (width 0.2) (layer "F.Cu") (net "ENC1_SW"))
 (segment (start 102.1962 100.0333) (end 102.1962 96.7038) (width 0.2) (layer "F.Cu") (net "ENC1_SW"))
 (segment (start 102.1962 96.7038) (end 103.91 94.99) (width 0.2) (layer "F.Cu") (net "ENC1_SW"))
 (segment (start 132.1806 101.1794) (end 103.3423 101.1794) (width 0.2) (layer "F.Cu") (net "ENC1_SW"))
 (segment (start 103.4781 98.8383) (end 103.91 98.8383) (width 0.2) (layer "F.Cu") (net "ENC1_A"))
 (segment (start 102.6123 96.991) (end 102.6123 97.9725) (width 0.2) (layer "F.Cu") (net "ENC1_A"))
 (segment (start 103.91 99.99) (end 103.91 98.8383) (width 0.2) (layer "F.Cu") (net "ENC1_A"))
 (segment (start 118.96 89.99) (end 117.9032 91.0468) (width 0.2) (layer "F.Cu") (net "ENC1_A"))
 (segment (start 134.48 103.96) (end 135.6453 102.7947) (width 0.2) (layer "F.Cu") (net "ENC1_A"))
 (segment (start 102.6123 97.9725) (end 103.4781 98.8383) (width 0.2) (layer "F.Cu") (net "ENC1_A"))
 (segment (start 135.0038 97.69) (end 124.713 97.69) (width 0.2) (layer "F.Cu") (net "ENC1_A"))
 (segment (start 123.5647 98.8383) (end 103.91 98.8383) (width 0.2) (layer "F.Cu") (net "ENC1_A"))
 (segment (start 108.6517 96.3358) (end 103.2675 96.3358) (width 0.2) (layer "F.Cu") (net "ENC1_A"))
 (segment (start 135.6453 98.3315) (end 135.0038 97.69) (width 0.2) (layer "F.Cu") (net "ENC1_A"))
 (segment (start 117.9032 91.0468) (end 116.0543 91.0468) (width 0.2) (layer "F.Cu") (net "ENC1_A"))
 (segment (start 124.713 97.69) (end 123.5647 98.8383) (width 0.2) (layer "F.Cu") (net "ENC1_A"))
 (segment (start 116.0543 91.0468) (end 114.9975 89.99) (width 0.2) (layer "F.Cu") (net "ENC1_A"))
 (segment (start 114.9975 89.99) (end 108.6517 96.3358) (width 0.2) (layer "F.Cu") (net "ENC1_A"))
 (segment (start 103.2675 96.3358) (end 102.6123 96.991) (width 0.2) (layer "F.Cu") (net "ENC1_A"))
 (segment (start 135.6453 102.7947) (end 135.6453 98.3315) (width 0.2) (layer "F.Cu") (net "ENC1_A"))
 (segment (start 101.766 102.1262) (end 101.766 95.024) (width 0.2) (layer "F.Cu") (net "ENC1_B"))
 (segment (start 130.91 104.99) (end 134.48 101.42) (width 0.2) (layer "F.Cu") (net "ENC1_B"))
 (segment (start 117.9386 83.9686) (end 118.96 84.99) (width 0.2) (layer "F.Cu") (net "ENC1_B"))
 (segment (start 116.0189 83.9686) (end 117.9386 83.9686) (width 0.2) (layer "F.Cu") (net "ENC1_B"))
 (segment (start 103.4781 103.8383) (end 101.766 102.1262) (width 0.2) (layer "F.Cu") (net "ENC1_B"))
 (segment (start 111.8 84.99) (end 114.9975 84.99) (width 0.2) (layer "F.Cu") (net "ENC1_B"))
 (segment (start 101.766 95.024) (end 111.8 84.99) (width 0.2) (layer "F.Cu") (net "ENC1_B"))
 (segment (start 103.91 104.99) (end 103.91 103.8383) (width 0.2) (layer "F.Cu") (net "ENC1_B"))
 (segment (start 103.91 104.99) (end 130.91 104.99) (width 0.2) (layer "F.Cu") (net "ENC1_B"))
 (segment (start 103.91 103.8383) (end 103.4781 103.8383) (width 0.2) (layer "F.Cu") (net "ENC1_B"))
 (segment (start 114.9975 84.99) (end 116.0189 83.9686) (width 0.2) (layer "F.Cu") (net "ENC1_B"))
 (segment (start 144.66 58.22) (end 134.48 68.4) (width 0.2) (layer "B.Cu") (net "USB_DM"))
 (segment (start 144.66 51.99) (end 144.66 58.22) (width 0.2) (layer "B.Cu") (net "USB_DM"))
 (segment (start 147.16 51.99) (end 147.16 58.26) (width 0.2) (layer "B.Cu") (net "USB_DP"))
 (segment (start 147.16 58.26) (end 134.48 70.94) (width 0.2) (layer "B.Cu") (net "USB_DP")))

